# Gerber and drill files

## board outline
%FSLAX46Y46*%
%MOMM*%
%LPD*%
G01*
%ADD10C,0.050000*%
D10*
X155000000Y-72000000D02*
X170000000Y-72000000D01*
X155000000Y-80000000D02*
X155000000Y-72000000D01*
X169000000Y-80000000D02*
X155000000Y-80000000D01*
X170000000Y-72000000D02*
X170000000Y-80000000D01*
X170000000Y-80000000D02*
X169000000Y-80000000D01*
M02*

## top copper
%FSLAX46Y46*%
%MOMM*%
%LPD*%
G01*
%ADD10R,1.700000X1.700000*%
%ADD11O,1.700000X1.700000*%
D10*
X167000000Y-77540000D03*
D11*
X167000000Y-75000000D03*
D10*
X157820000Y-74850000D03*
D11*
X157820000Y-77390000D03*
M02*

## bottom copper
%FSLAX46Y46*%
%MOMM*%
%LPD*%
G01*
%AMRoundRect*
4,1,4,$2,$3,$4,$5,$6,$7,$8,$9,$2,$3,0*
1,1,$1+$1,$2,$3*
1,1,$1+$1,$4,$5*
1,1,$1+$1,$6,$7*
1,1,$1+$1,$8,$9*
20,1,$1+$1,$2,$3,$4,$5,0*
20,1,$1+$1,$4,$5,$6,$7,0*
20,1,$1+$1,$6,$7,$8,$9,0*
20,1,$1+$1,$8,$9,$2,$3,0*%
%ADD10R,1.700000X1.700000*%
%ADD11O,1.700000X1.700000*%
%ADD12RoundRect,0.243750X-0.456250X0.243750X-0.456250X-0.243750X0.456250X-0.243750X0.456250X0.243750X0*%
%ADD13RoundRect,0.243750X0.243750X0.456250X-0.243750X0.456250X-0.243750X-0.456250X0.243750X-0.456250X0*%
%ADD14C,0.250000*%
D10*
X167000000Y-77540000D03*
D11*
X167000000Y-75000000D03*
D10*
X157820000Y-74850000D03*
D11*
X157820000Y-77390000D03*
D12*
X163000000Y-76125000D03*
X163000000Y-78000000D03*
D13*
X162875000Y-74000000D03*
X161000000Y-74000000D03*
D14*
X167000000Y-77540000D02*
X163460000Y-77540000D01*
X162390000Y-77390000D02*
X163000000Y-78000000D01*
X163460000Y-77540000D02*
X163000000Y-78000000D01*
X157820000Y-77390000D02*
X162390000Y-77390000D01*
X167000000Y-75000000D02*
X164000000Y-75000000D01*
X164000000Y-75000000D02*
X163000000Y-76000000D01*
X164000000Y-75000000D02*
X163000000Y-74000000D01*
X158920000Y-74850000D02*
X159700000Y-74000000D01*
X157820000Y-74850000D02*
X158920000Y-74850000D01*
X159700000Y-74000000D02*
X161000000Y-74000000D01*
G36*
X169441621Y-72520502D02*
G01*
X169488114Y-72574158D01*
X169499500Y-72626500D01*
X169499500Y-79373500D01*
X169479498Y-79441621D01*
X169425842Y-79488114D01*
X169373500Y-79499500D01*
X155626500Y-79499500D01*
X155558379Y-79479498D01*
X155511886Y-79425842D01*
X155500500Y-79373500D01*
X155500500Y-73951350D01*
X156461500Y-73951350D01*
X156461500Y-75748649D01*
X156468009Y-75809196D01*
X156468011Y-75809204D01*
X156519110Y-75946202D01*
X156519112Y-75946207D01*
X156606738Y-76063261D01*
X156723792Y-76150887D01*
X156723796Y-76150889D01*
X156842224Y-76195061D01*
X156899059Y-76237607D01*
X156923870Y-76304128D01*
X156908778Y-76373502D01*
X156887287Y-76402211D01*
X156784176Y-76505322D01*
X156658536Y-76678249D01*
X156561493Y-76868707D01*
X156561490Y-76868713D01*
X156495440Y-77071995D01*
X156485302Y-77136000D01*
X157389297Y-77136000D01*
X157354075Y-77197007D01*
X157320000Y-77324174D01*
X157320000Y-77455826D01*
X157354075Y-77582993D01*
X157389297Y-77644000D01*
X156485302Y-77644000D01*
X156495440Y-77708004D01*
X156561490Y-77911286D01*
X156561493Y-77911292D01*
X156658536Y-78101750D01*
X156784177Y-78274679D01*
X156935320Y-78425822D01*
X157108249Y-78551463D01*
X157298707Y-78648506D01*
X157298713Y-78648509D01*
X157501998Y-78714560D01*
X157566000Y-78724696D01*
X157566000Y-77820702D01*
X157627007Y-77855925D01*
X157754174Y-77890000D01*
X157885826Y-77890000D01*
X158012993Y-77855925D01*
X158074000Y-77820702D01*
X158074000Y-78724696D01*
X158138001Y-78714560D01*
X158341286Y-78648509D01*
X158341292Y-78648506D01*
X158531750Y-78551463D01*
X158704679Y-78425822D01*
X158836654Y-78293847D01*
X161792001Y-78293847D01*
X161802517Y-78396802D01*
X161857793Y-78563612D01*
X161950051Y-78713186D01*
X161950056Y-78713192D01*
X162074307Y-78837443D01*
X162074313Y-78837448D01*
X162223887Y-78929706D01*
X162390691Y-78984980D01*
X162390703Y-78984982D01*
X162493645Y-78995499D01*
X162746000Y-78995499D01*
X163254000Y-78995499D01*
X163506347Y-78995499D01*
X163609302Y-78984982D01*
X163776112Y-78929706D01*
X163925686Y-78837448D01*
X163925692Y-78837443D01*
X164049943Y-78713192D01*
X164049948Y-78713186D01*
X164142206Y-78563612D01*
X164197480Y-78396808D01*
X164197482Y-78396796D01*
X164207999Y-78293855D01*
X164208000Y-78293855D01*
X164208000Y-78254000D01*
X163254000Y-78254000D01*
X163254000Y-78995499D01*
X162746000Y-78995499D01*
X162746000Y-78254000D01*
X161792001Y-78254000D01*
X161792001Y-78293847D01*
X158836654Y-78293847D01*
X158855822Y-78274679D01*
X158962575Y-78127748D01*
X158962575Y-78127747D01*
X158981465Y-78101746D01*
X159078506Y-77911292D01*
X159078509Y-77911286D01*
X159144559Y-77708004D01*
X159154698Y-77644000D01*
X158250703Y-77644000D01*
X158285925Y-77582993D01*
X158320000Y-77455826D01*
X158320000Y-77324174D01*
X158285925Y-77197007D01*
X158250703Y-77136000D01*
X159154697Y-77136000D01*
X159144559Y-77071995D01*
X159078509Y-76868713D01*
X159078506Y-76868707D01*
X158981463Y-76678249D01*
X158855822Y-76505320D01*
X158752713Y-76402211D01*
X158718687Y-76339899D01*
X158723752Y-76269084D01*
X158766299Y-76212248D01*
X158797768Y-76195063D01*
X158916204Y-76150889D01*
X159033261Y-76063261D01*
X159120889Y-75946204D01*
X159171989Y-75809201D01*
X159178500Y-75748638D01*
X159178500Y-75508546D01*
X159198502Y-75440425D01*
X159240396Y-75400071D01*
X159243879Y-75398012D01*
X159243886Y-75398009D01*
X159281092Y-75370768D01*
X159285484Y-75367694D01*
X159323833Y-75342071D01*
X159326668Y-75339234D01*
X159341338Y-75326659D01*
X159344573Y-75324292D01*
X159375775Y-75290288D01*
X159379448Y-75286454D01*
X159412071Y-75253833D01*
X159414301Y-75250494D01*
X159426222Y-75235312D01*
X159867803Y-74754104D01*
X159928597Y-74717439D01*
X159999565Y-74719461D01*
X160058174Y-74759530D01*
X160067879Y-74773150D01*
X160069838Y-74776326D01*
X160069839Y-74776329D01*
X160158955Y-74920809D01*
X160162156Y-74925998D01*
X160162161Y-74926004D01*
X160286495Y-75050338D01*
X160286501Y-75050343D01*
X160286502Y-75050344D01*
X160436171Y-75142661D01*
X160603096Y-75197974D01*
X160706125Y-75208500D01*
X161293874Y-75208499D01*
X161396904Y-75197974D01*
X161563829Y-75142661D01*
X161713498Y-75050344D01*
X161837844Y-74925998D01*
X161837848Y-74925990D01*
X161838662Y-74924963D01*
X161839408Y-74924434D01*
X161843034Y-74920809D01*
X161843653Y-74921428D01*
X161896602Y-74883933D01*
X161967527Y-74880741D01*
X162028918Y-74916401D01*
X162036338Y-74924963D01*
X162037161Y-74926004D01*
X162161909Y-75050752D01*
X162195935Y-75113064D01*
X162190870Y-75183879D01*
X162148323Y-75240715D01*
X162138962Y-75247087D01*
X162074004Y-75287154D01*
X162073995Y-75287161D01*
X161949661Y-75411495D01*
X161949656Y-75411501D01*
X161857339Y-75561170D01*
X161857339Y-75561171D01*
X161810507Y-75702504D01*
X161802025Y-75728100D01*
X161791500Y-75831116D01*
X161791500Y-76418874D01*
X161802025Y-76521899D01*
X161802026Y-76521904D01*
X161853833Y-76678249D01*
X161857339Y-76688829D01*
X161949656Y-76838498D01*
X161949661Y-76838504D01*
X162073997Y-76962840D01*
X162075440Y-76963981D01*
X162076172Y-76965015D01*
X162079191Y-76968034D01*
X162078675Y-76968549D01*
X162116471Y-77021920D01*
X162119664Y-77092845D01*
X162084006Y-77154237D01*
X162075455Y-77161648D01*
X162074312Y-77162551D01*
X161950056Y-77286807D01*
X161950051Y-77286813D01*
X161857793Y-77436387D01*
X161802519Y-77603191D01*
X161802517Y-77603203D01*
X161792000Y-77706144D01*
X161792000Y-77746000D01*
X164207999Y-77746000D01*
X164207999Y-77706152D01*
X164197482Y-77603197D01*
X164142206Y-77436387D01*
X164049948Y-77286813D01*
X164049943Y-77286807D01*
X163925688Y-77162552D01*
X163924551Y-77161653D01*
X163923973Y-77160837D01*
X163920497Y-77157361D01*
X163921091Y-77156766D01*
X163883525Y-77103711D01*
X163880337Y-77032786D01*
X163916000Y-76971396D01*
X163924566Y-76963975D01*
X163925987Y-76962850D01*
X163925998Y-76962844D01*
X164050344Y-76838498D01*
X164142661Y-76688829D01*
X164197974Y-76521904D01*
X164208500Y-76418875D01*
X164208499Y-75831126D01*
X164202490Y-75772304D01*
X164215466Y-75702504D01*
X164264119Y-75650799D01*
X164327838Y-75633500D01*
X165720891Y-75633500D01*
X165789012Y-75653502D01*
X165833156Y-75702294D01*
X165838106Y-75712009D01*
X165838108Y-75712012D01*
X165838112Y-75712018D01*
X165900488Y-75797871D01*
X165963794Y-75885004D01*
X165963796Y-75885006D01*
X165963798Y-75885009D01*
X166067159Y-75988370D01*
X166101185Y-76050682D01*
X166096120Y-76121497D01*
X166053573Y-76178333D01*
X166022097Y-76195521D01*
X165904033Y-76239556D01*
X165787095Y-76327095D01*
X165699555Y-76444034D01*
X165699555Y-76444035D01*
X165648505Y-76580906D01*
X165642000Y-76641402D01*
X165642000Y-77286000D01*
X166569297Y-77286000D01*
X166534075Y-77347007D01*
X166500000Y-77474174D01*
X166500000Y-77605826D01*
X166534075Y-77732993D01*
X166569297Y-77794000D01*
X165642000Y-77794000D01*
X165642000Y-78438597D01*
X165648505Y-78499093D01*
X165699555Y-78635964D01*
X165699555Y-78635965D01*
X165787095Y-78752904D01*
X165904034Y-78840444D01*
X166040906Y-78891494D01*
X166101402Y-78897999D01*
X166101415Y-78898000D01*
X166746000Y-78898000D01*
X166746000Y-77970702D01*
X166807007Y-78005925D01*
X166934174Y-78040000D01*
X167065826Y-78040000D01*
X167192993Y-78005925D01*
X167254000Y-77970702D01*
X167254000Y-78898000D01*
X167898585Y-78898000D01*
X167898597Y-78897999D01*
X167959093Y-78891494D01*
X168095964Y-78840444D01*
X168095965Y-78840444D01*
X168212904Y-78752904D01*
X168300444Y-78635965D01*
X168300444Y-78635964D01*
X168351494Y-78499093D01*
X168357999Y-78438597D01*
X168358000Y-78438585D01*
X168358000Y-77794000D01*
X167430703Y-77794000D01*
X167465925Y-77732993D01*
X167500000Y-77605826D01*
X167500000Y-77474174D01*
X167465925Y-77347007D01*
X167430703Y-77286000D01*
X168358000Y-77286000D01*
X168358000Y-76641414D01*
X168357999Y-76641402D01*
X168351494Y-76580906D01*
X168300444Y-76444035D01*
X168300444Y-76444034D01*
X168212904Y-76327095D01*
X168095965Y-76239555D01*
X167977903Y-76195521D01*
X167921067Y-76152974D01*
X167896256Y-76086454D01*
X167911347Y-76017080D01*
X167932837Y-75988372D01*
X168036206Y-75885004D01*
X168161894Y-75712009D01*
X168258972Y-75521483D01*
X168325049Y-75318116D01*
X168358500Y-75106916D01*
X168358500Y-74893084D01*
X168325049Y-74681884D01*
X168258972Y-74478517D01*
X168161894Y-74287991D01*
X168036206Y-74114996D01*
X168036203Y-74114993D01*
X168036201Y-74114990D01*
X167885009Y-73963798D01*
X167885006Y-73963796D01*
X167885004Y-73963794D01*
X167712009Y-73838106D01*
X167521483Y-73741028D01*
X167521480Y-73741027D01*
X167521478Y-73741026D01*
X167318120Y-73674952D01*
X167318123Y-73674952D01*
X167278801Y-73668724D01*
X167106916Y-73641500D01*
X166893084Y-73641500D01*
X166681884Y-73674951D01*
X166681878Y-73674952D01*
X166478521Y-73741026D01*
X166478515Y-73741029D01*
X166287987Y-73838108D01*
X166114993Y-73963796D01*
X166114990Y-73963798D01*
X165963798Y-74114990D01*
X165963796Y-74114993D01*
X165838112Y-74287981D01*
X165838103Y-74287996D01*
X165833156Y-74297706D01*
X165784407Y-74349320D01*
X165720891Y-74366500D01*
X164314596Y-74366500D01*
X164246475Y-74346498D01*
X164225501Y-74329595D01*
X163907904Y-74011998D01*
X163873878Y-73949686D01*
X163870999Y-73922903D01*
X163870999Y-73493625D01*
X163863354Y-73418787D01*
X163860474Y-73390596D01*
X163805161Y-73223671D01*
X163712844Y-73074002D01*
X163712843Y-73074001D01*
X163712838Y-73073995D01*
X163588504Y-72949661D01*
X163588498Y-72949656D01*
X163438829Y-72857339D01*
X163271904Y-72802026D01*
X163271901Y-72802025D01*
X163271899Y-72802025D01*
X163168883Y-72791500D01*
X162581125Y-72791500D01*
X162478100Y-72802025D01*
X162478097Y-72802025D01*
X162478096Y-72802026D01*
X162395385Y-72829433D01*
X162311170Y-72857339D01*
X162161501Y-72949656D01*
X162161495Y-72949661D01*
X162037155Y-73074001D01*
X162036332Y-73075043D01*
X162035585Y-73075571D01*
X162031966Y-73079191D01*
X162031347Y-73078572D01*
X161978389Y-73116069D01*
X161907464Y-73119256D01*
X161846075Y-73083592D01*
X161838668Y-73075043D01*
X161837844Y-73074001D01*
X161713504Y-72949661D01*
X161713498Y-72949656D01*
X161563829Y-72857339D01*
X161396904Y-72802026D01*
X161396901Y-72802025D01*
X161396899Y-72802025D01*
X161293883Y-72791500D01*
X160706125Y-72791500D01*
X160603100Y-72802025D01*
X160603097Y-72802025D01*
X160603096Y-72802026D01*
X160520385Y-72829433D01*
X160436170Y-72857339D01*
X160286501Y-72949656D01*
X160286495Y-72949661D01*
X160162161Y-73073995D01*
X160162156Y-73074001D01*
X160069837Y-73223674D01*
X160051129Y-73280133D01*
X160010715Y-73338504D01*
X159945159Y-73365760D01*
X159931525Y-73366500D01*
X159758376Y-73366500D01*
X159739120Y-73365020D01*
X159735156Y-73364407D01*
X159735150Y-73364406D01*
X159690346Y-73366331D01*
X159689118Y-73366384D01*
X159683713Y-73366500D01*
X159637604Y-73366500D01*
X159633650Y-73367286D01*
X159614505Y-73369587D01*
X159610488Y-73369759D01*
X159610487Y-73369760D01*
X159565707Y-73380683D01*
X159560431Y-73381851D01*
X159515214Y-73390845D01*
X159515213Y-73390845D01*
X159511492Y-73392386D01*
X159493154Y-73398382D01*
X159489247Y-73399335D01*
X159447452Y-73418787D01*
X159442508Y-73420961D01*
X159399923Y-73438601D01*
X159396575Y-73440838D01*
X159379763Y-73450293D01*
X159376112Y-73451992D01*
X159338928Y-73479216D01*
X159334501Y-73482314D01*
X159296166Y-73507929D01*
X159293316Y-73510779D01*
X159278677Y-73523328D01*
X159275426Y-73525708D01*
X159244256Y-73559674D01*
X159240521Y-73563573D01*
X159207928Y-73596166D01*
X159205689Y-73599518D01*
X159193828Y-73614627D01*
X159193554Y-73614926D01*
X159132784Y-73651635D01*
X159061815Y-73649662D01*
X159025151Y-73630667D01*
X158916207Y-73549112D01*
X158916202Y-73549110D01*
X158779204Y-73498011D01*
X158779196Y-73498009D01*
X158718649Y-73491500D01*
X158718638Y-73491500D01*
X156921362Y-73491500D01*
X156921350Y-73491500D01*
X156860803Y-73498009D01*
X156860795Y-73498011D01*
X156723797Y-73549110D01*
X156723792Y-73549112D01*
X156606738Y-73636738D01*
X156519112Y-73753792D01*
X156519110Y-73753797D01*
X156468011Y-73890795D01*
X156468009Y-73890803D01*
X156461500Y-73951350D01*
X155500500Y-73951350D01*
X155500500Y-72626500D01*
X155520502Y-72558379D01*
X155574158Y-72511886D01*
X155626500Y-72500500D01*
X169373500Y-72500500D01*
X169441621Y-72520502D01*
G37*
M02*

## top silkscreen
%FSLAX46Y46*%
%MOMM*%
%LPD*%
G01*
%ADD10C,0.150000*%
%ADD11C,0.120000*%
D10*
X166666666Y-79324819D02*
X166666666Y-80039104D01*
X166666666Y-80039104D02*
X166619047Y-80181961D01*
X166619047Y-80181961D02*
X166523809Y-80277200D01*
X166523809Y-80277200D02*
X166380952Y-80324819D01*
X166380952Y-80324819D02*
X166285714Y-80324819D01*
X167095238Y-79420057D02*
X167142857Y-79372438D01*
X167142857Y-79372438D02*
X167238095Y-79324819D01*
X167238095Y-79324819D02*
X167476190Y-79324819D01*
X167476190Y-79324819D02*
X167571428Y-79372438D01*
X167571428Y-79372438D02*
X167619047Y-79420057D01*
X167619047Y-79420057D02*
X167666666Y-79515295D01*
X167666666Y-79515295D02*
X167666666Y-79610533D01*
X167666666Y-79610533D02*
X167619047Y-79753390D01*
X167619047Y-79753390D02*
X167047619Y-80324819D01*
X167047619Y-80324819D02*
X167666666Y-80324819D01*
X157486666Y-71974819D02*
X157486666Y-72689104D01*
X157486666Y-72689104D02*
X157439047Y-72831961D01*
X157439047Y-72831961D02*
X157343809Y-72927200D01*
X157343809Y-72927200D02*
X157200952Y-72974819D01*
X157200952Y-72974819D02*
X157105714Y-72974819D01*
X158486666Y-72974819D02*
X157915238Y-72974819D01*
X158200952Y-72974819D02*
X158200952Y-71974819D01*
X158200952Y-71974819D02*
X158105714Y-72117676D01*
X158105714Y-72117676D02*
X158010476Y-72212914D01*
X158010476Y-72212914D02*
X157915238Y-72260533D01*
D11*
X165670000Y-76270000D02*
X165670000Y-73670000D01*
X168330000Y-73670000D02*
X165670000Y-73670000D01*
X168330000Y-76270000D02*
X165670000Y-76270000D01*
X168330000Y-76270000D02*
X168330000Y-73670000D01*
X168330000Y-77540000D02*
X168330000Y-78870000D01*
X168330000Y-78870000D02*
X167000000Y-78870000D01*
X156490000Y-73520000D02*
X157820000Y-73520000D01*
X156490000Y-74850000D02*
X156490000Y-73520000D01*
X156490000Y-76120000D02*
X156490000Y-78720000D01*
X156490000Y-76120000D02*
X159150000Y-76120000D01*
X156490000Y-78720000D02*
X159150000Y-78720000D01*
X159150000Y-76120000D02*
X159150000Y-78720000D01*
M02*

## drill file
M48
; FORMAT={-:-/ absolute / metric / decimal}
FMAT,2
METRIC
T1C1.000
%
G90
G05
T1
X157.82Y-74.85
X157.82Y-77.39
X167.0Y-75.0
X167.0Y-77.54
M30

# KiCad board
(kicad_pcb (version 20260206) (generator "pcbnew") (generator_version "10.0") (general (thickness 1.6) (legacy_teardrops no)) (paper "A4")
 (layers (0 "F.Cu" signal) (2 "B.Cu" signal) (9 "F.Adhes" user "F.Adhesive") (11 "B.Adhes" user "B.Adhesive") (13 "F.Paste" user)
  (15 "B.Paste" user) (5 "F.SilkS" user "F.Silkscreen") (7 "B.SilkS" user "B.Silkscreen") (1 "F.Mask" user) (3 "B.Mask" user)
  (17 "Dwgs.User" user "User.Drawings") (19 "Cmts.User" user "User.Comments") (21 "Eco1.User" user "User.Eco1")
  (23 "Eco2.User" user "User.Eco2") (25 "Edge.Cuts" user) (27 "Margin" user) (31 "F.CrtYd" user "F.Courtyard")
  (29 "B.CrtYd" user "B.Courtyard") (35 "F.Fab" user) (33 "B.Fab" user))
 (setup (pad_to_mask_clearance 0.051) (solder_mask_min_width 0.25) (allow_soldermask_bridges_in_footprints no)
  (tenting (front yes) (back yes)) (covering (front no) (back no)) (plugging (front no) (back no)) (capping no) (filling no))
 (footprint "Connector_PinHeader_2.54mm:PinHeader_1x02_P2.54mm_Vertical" (layer "F.Cu") (at 167 77.54 180)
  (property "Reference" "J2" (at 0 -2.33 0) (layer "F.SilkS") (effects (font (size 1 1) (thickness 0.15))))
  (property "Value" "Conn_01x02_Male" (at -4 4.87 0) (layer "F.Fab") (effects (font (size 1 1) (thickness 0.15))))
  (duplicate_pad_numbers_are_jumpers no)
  (fp_line (start 1.33 1.27) (end 1.33 3.87) (stroke (width 0.12) (type solid)) (layer "F.SilkS"))
  (fp_line (start -1.33 3.87) (end 1.33 3.87) (stroke (width 0.12) (type solid)) (layer "F.SilkS"))
  (fp_line (start -1.33 1.27) (end 1.33 1.27) (stroke (width 0.12) (type solid)) (layer "F.SilkS"))
  (fp_line (start -1.33 1.27) (end -1.33 3.87) (stroke (width 0.12) (type solid)) (layer "F.SilkS"))
  (fp_line (start -1.33 0) (end -1.33 -1.33) (stroke (width 0.12) (type solid)) (layer "F.SilkS"))
  (fp_line (start -1.33 -1.33) (end 0 -1.33) (stroke (width 0.12) (type solid)) (layer "F.SilkS"))
  (pad "1" thru_hole rect (at 0 0 180) (size 1.7 1.7) (drill 1) (layers "*.Cu" "*.Mask") (remove_unused_layers no) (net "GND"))
  (pad "2" thru_hole oval (at 0 2.54 180) (size 1.7 1.7) (drill 1) (layers "*.Cu" "*.Mask") (remove_unused_layers no) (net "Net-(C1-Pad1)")))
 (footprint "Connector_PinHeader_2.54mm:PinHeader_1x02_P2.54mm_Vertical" (layer "F.Cu") (at 157.82 74.85)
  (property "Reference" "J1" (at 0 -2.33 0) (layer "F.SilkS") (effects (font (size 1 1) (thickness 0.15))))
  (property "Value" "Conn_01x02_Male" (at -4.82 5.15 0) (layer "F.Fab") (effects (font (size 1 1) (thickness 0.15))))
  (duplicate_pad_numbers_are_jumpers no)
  (fp_line (start -1.33 -1.33) (end 0 -1.33) (stroke (width 0.12) (type solid)) (layer "F.SilkS"))
  (fp_line (start -1.33 0) (end -1.33 -1.33) (stroke (width 0.12) (type solid)) (layer "F.SilkS"))
  (fp_line (start -1.33 1.27) (end -1.33 3.87) (stroke (width 0.12) (type solid)) (layer "F.SilkS"))
  (fp_line (start -1.33 1.27) (end 1.33 1.27) (stroke (width 0.12) (type solid)) (layer "F.SilkS"))
  (fp_line (start -1.33 3.87) (end 1.33 3.87) (stroke (width 0.12) (type solid)) (layer "F.SilkS"))
  (fp_line (start 1.33 1.27) (end 1.33 3.87) (stroke (width 0.12) (type solid)) (layer "F.SilkS"))
  (pad "1" thru_hole rect (at 0 0) (size 1.7 1.7) (drill 1) (layers "*.Cu" "*.Mask") (remove_unused_layers no) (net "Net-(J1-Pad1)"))
  (pad "2" thru_hole oval (at 0 2.54) (size 1.7 1.7) (drill 1) (layers "*.Cu" "*.Mask") (remove_unused_layers no) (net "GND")))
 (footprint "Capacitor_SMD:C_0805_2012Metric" (layer "B.Cu") (at 163 77.0625 -90)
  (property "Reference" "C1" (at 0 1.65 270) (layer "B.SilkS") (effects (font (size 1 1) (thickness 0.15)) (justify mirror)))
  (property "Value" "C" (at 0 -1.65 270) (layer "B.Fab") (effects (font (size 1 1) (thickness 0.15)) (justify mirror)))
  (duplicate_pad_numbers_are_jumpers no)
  (pad "1" smd roundrect (at -0.9375 0 270) (size 0.975 1.4) (layers "B.Cu" "B.Mask" "B.Paste") (roundrect_rratio 0.25)
   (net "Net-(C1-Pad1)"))
  (pad "2" smd roundrect (at 0.9375 0 270) (size 0.975 1.4) (layers "B.Cu" "B.Mask" "B.Paste") (roundrect_rratio 0.25) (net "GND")))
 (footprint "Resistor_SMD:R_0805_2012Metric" (layer "B.Cu") (at 161.9375 74 180)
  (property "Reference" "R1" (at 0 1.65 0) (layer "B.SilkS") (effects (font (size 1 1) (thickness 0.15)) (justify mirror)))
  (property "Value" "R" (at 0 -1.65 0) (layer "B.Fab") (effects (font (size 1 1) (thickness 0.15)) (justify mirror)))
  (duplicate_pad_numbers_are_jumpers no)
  (pad "1" smd roundrect (at -0.9375 0 180) (size 0.975 1.4) (layers "B.Cu" "B.Mask" "B.Paste") (roundrect_rratio 0.25)
   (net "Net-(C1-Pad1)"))
  (pad "2" smd roundrect (at 0.9375 0 180) (size 0.975 1.4) (layers "B.Cu" "B.Mask" "B.Paste") (roundrect_rratio 0.25) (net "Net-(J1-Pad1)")))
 (gr_line (start 155 72) (end 170 72) (stroke (width 0.05) (type solid)) (layer "Edge.Cuts"))
 (gr_line (start 155 80) (end 155 72) (stroke (width 0.05) (type solid)) (layer "Edge.Cuts"))
 (gr_line (start 169 80) (end 155 80) (stroke (width 0.05) (type solid)) (layer "Edge.Cuts"))
 (gr_line (start 170 72) (end 170 80) (stroke (width 0.05) (type solid)) (layer "Edge.Cuts"))
 (gr_line (start 170 80) (end 169 80) (stroke (width 0.05) (type solid)) (layer "Edge.Cuts"))
 (segment (start 167 77.54) (end 163.46 77.54) (width 0.25) (layer "B.Cu") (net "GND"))
 (segment (start 162.39 77.39) (end 163 78) (width 0.25) (layer "B.Cu") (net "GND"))
 (segment (start 163.46 77.54) (end 163 78) (width 0.25) (layer "B.Cu") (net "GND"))
 (segment (start 157.82 77.39) (end 162.39 77.39) (width 0.25) (layer "B.Cu") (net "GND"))
 (segment (start 167 75) (end 164 75) (width 0.25) (layer "B.Cu") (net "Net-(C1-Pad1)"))
 (segment (start 164 75) (end 163 76) (width 0.25) (layer "B.Cu") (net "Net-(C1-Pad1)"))
 (segment (start 164 75) (end 163 74) (width 0.25) (layer "B.Cu") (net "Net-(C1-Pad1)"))
 (segment (start 158.92 74.85) (end 159.7 74) (width 0.25) (layer "B.Cu") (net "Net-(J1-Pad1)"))
 (segment (start 157.82 74.85) (end 158.92 74.85) (width 0.25) (layer "B.Cu") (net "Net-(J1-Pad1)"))
 (segment (start 159.7 74) (end 161 74) (width 0.25) (layer "B.Cu") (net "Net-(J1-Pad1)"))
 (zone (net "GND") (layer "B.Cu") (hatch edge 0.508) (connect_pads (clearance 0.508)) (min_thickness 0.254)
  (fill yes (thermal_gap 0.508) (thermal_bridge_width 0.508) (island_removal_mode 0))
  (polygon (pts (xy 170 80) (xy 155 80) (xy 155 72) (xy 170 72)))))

